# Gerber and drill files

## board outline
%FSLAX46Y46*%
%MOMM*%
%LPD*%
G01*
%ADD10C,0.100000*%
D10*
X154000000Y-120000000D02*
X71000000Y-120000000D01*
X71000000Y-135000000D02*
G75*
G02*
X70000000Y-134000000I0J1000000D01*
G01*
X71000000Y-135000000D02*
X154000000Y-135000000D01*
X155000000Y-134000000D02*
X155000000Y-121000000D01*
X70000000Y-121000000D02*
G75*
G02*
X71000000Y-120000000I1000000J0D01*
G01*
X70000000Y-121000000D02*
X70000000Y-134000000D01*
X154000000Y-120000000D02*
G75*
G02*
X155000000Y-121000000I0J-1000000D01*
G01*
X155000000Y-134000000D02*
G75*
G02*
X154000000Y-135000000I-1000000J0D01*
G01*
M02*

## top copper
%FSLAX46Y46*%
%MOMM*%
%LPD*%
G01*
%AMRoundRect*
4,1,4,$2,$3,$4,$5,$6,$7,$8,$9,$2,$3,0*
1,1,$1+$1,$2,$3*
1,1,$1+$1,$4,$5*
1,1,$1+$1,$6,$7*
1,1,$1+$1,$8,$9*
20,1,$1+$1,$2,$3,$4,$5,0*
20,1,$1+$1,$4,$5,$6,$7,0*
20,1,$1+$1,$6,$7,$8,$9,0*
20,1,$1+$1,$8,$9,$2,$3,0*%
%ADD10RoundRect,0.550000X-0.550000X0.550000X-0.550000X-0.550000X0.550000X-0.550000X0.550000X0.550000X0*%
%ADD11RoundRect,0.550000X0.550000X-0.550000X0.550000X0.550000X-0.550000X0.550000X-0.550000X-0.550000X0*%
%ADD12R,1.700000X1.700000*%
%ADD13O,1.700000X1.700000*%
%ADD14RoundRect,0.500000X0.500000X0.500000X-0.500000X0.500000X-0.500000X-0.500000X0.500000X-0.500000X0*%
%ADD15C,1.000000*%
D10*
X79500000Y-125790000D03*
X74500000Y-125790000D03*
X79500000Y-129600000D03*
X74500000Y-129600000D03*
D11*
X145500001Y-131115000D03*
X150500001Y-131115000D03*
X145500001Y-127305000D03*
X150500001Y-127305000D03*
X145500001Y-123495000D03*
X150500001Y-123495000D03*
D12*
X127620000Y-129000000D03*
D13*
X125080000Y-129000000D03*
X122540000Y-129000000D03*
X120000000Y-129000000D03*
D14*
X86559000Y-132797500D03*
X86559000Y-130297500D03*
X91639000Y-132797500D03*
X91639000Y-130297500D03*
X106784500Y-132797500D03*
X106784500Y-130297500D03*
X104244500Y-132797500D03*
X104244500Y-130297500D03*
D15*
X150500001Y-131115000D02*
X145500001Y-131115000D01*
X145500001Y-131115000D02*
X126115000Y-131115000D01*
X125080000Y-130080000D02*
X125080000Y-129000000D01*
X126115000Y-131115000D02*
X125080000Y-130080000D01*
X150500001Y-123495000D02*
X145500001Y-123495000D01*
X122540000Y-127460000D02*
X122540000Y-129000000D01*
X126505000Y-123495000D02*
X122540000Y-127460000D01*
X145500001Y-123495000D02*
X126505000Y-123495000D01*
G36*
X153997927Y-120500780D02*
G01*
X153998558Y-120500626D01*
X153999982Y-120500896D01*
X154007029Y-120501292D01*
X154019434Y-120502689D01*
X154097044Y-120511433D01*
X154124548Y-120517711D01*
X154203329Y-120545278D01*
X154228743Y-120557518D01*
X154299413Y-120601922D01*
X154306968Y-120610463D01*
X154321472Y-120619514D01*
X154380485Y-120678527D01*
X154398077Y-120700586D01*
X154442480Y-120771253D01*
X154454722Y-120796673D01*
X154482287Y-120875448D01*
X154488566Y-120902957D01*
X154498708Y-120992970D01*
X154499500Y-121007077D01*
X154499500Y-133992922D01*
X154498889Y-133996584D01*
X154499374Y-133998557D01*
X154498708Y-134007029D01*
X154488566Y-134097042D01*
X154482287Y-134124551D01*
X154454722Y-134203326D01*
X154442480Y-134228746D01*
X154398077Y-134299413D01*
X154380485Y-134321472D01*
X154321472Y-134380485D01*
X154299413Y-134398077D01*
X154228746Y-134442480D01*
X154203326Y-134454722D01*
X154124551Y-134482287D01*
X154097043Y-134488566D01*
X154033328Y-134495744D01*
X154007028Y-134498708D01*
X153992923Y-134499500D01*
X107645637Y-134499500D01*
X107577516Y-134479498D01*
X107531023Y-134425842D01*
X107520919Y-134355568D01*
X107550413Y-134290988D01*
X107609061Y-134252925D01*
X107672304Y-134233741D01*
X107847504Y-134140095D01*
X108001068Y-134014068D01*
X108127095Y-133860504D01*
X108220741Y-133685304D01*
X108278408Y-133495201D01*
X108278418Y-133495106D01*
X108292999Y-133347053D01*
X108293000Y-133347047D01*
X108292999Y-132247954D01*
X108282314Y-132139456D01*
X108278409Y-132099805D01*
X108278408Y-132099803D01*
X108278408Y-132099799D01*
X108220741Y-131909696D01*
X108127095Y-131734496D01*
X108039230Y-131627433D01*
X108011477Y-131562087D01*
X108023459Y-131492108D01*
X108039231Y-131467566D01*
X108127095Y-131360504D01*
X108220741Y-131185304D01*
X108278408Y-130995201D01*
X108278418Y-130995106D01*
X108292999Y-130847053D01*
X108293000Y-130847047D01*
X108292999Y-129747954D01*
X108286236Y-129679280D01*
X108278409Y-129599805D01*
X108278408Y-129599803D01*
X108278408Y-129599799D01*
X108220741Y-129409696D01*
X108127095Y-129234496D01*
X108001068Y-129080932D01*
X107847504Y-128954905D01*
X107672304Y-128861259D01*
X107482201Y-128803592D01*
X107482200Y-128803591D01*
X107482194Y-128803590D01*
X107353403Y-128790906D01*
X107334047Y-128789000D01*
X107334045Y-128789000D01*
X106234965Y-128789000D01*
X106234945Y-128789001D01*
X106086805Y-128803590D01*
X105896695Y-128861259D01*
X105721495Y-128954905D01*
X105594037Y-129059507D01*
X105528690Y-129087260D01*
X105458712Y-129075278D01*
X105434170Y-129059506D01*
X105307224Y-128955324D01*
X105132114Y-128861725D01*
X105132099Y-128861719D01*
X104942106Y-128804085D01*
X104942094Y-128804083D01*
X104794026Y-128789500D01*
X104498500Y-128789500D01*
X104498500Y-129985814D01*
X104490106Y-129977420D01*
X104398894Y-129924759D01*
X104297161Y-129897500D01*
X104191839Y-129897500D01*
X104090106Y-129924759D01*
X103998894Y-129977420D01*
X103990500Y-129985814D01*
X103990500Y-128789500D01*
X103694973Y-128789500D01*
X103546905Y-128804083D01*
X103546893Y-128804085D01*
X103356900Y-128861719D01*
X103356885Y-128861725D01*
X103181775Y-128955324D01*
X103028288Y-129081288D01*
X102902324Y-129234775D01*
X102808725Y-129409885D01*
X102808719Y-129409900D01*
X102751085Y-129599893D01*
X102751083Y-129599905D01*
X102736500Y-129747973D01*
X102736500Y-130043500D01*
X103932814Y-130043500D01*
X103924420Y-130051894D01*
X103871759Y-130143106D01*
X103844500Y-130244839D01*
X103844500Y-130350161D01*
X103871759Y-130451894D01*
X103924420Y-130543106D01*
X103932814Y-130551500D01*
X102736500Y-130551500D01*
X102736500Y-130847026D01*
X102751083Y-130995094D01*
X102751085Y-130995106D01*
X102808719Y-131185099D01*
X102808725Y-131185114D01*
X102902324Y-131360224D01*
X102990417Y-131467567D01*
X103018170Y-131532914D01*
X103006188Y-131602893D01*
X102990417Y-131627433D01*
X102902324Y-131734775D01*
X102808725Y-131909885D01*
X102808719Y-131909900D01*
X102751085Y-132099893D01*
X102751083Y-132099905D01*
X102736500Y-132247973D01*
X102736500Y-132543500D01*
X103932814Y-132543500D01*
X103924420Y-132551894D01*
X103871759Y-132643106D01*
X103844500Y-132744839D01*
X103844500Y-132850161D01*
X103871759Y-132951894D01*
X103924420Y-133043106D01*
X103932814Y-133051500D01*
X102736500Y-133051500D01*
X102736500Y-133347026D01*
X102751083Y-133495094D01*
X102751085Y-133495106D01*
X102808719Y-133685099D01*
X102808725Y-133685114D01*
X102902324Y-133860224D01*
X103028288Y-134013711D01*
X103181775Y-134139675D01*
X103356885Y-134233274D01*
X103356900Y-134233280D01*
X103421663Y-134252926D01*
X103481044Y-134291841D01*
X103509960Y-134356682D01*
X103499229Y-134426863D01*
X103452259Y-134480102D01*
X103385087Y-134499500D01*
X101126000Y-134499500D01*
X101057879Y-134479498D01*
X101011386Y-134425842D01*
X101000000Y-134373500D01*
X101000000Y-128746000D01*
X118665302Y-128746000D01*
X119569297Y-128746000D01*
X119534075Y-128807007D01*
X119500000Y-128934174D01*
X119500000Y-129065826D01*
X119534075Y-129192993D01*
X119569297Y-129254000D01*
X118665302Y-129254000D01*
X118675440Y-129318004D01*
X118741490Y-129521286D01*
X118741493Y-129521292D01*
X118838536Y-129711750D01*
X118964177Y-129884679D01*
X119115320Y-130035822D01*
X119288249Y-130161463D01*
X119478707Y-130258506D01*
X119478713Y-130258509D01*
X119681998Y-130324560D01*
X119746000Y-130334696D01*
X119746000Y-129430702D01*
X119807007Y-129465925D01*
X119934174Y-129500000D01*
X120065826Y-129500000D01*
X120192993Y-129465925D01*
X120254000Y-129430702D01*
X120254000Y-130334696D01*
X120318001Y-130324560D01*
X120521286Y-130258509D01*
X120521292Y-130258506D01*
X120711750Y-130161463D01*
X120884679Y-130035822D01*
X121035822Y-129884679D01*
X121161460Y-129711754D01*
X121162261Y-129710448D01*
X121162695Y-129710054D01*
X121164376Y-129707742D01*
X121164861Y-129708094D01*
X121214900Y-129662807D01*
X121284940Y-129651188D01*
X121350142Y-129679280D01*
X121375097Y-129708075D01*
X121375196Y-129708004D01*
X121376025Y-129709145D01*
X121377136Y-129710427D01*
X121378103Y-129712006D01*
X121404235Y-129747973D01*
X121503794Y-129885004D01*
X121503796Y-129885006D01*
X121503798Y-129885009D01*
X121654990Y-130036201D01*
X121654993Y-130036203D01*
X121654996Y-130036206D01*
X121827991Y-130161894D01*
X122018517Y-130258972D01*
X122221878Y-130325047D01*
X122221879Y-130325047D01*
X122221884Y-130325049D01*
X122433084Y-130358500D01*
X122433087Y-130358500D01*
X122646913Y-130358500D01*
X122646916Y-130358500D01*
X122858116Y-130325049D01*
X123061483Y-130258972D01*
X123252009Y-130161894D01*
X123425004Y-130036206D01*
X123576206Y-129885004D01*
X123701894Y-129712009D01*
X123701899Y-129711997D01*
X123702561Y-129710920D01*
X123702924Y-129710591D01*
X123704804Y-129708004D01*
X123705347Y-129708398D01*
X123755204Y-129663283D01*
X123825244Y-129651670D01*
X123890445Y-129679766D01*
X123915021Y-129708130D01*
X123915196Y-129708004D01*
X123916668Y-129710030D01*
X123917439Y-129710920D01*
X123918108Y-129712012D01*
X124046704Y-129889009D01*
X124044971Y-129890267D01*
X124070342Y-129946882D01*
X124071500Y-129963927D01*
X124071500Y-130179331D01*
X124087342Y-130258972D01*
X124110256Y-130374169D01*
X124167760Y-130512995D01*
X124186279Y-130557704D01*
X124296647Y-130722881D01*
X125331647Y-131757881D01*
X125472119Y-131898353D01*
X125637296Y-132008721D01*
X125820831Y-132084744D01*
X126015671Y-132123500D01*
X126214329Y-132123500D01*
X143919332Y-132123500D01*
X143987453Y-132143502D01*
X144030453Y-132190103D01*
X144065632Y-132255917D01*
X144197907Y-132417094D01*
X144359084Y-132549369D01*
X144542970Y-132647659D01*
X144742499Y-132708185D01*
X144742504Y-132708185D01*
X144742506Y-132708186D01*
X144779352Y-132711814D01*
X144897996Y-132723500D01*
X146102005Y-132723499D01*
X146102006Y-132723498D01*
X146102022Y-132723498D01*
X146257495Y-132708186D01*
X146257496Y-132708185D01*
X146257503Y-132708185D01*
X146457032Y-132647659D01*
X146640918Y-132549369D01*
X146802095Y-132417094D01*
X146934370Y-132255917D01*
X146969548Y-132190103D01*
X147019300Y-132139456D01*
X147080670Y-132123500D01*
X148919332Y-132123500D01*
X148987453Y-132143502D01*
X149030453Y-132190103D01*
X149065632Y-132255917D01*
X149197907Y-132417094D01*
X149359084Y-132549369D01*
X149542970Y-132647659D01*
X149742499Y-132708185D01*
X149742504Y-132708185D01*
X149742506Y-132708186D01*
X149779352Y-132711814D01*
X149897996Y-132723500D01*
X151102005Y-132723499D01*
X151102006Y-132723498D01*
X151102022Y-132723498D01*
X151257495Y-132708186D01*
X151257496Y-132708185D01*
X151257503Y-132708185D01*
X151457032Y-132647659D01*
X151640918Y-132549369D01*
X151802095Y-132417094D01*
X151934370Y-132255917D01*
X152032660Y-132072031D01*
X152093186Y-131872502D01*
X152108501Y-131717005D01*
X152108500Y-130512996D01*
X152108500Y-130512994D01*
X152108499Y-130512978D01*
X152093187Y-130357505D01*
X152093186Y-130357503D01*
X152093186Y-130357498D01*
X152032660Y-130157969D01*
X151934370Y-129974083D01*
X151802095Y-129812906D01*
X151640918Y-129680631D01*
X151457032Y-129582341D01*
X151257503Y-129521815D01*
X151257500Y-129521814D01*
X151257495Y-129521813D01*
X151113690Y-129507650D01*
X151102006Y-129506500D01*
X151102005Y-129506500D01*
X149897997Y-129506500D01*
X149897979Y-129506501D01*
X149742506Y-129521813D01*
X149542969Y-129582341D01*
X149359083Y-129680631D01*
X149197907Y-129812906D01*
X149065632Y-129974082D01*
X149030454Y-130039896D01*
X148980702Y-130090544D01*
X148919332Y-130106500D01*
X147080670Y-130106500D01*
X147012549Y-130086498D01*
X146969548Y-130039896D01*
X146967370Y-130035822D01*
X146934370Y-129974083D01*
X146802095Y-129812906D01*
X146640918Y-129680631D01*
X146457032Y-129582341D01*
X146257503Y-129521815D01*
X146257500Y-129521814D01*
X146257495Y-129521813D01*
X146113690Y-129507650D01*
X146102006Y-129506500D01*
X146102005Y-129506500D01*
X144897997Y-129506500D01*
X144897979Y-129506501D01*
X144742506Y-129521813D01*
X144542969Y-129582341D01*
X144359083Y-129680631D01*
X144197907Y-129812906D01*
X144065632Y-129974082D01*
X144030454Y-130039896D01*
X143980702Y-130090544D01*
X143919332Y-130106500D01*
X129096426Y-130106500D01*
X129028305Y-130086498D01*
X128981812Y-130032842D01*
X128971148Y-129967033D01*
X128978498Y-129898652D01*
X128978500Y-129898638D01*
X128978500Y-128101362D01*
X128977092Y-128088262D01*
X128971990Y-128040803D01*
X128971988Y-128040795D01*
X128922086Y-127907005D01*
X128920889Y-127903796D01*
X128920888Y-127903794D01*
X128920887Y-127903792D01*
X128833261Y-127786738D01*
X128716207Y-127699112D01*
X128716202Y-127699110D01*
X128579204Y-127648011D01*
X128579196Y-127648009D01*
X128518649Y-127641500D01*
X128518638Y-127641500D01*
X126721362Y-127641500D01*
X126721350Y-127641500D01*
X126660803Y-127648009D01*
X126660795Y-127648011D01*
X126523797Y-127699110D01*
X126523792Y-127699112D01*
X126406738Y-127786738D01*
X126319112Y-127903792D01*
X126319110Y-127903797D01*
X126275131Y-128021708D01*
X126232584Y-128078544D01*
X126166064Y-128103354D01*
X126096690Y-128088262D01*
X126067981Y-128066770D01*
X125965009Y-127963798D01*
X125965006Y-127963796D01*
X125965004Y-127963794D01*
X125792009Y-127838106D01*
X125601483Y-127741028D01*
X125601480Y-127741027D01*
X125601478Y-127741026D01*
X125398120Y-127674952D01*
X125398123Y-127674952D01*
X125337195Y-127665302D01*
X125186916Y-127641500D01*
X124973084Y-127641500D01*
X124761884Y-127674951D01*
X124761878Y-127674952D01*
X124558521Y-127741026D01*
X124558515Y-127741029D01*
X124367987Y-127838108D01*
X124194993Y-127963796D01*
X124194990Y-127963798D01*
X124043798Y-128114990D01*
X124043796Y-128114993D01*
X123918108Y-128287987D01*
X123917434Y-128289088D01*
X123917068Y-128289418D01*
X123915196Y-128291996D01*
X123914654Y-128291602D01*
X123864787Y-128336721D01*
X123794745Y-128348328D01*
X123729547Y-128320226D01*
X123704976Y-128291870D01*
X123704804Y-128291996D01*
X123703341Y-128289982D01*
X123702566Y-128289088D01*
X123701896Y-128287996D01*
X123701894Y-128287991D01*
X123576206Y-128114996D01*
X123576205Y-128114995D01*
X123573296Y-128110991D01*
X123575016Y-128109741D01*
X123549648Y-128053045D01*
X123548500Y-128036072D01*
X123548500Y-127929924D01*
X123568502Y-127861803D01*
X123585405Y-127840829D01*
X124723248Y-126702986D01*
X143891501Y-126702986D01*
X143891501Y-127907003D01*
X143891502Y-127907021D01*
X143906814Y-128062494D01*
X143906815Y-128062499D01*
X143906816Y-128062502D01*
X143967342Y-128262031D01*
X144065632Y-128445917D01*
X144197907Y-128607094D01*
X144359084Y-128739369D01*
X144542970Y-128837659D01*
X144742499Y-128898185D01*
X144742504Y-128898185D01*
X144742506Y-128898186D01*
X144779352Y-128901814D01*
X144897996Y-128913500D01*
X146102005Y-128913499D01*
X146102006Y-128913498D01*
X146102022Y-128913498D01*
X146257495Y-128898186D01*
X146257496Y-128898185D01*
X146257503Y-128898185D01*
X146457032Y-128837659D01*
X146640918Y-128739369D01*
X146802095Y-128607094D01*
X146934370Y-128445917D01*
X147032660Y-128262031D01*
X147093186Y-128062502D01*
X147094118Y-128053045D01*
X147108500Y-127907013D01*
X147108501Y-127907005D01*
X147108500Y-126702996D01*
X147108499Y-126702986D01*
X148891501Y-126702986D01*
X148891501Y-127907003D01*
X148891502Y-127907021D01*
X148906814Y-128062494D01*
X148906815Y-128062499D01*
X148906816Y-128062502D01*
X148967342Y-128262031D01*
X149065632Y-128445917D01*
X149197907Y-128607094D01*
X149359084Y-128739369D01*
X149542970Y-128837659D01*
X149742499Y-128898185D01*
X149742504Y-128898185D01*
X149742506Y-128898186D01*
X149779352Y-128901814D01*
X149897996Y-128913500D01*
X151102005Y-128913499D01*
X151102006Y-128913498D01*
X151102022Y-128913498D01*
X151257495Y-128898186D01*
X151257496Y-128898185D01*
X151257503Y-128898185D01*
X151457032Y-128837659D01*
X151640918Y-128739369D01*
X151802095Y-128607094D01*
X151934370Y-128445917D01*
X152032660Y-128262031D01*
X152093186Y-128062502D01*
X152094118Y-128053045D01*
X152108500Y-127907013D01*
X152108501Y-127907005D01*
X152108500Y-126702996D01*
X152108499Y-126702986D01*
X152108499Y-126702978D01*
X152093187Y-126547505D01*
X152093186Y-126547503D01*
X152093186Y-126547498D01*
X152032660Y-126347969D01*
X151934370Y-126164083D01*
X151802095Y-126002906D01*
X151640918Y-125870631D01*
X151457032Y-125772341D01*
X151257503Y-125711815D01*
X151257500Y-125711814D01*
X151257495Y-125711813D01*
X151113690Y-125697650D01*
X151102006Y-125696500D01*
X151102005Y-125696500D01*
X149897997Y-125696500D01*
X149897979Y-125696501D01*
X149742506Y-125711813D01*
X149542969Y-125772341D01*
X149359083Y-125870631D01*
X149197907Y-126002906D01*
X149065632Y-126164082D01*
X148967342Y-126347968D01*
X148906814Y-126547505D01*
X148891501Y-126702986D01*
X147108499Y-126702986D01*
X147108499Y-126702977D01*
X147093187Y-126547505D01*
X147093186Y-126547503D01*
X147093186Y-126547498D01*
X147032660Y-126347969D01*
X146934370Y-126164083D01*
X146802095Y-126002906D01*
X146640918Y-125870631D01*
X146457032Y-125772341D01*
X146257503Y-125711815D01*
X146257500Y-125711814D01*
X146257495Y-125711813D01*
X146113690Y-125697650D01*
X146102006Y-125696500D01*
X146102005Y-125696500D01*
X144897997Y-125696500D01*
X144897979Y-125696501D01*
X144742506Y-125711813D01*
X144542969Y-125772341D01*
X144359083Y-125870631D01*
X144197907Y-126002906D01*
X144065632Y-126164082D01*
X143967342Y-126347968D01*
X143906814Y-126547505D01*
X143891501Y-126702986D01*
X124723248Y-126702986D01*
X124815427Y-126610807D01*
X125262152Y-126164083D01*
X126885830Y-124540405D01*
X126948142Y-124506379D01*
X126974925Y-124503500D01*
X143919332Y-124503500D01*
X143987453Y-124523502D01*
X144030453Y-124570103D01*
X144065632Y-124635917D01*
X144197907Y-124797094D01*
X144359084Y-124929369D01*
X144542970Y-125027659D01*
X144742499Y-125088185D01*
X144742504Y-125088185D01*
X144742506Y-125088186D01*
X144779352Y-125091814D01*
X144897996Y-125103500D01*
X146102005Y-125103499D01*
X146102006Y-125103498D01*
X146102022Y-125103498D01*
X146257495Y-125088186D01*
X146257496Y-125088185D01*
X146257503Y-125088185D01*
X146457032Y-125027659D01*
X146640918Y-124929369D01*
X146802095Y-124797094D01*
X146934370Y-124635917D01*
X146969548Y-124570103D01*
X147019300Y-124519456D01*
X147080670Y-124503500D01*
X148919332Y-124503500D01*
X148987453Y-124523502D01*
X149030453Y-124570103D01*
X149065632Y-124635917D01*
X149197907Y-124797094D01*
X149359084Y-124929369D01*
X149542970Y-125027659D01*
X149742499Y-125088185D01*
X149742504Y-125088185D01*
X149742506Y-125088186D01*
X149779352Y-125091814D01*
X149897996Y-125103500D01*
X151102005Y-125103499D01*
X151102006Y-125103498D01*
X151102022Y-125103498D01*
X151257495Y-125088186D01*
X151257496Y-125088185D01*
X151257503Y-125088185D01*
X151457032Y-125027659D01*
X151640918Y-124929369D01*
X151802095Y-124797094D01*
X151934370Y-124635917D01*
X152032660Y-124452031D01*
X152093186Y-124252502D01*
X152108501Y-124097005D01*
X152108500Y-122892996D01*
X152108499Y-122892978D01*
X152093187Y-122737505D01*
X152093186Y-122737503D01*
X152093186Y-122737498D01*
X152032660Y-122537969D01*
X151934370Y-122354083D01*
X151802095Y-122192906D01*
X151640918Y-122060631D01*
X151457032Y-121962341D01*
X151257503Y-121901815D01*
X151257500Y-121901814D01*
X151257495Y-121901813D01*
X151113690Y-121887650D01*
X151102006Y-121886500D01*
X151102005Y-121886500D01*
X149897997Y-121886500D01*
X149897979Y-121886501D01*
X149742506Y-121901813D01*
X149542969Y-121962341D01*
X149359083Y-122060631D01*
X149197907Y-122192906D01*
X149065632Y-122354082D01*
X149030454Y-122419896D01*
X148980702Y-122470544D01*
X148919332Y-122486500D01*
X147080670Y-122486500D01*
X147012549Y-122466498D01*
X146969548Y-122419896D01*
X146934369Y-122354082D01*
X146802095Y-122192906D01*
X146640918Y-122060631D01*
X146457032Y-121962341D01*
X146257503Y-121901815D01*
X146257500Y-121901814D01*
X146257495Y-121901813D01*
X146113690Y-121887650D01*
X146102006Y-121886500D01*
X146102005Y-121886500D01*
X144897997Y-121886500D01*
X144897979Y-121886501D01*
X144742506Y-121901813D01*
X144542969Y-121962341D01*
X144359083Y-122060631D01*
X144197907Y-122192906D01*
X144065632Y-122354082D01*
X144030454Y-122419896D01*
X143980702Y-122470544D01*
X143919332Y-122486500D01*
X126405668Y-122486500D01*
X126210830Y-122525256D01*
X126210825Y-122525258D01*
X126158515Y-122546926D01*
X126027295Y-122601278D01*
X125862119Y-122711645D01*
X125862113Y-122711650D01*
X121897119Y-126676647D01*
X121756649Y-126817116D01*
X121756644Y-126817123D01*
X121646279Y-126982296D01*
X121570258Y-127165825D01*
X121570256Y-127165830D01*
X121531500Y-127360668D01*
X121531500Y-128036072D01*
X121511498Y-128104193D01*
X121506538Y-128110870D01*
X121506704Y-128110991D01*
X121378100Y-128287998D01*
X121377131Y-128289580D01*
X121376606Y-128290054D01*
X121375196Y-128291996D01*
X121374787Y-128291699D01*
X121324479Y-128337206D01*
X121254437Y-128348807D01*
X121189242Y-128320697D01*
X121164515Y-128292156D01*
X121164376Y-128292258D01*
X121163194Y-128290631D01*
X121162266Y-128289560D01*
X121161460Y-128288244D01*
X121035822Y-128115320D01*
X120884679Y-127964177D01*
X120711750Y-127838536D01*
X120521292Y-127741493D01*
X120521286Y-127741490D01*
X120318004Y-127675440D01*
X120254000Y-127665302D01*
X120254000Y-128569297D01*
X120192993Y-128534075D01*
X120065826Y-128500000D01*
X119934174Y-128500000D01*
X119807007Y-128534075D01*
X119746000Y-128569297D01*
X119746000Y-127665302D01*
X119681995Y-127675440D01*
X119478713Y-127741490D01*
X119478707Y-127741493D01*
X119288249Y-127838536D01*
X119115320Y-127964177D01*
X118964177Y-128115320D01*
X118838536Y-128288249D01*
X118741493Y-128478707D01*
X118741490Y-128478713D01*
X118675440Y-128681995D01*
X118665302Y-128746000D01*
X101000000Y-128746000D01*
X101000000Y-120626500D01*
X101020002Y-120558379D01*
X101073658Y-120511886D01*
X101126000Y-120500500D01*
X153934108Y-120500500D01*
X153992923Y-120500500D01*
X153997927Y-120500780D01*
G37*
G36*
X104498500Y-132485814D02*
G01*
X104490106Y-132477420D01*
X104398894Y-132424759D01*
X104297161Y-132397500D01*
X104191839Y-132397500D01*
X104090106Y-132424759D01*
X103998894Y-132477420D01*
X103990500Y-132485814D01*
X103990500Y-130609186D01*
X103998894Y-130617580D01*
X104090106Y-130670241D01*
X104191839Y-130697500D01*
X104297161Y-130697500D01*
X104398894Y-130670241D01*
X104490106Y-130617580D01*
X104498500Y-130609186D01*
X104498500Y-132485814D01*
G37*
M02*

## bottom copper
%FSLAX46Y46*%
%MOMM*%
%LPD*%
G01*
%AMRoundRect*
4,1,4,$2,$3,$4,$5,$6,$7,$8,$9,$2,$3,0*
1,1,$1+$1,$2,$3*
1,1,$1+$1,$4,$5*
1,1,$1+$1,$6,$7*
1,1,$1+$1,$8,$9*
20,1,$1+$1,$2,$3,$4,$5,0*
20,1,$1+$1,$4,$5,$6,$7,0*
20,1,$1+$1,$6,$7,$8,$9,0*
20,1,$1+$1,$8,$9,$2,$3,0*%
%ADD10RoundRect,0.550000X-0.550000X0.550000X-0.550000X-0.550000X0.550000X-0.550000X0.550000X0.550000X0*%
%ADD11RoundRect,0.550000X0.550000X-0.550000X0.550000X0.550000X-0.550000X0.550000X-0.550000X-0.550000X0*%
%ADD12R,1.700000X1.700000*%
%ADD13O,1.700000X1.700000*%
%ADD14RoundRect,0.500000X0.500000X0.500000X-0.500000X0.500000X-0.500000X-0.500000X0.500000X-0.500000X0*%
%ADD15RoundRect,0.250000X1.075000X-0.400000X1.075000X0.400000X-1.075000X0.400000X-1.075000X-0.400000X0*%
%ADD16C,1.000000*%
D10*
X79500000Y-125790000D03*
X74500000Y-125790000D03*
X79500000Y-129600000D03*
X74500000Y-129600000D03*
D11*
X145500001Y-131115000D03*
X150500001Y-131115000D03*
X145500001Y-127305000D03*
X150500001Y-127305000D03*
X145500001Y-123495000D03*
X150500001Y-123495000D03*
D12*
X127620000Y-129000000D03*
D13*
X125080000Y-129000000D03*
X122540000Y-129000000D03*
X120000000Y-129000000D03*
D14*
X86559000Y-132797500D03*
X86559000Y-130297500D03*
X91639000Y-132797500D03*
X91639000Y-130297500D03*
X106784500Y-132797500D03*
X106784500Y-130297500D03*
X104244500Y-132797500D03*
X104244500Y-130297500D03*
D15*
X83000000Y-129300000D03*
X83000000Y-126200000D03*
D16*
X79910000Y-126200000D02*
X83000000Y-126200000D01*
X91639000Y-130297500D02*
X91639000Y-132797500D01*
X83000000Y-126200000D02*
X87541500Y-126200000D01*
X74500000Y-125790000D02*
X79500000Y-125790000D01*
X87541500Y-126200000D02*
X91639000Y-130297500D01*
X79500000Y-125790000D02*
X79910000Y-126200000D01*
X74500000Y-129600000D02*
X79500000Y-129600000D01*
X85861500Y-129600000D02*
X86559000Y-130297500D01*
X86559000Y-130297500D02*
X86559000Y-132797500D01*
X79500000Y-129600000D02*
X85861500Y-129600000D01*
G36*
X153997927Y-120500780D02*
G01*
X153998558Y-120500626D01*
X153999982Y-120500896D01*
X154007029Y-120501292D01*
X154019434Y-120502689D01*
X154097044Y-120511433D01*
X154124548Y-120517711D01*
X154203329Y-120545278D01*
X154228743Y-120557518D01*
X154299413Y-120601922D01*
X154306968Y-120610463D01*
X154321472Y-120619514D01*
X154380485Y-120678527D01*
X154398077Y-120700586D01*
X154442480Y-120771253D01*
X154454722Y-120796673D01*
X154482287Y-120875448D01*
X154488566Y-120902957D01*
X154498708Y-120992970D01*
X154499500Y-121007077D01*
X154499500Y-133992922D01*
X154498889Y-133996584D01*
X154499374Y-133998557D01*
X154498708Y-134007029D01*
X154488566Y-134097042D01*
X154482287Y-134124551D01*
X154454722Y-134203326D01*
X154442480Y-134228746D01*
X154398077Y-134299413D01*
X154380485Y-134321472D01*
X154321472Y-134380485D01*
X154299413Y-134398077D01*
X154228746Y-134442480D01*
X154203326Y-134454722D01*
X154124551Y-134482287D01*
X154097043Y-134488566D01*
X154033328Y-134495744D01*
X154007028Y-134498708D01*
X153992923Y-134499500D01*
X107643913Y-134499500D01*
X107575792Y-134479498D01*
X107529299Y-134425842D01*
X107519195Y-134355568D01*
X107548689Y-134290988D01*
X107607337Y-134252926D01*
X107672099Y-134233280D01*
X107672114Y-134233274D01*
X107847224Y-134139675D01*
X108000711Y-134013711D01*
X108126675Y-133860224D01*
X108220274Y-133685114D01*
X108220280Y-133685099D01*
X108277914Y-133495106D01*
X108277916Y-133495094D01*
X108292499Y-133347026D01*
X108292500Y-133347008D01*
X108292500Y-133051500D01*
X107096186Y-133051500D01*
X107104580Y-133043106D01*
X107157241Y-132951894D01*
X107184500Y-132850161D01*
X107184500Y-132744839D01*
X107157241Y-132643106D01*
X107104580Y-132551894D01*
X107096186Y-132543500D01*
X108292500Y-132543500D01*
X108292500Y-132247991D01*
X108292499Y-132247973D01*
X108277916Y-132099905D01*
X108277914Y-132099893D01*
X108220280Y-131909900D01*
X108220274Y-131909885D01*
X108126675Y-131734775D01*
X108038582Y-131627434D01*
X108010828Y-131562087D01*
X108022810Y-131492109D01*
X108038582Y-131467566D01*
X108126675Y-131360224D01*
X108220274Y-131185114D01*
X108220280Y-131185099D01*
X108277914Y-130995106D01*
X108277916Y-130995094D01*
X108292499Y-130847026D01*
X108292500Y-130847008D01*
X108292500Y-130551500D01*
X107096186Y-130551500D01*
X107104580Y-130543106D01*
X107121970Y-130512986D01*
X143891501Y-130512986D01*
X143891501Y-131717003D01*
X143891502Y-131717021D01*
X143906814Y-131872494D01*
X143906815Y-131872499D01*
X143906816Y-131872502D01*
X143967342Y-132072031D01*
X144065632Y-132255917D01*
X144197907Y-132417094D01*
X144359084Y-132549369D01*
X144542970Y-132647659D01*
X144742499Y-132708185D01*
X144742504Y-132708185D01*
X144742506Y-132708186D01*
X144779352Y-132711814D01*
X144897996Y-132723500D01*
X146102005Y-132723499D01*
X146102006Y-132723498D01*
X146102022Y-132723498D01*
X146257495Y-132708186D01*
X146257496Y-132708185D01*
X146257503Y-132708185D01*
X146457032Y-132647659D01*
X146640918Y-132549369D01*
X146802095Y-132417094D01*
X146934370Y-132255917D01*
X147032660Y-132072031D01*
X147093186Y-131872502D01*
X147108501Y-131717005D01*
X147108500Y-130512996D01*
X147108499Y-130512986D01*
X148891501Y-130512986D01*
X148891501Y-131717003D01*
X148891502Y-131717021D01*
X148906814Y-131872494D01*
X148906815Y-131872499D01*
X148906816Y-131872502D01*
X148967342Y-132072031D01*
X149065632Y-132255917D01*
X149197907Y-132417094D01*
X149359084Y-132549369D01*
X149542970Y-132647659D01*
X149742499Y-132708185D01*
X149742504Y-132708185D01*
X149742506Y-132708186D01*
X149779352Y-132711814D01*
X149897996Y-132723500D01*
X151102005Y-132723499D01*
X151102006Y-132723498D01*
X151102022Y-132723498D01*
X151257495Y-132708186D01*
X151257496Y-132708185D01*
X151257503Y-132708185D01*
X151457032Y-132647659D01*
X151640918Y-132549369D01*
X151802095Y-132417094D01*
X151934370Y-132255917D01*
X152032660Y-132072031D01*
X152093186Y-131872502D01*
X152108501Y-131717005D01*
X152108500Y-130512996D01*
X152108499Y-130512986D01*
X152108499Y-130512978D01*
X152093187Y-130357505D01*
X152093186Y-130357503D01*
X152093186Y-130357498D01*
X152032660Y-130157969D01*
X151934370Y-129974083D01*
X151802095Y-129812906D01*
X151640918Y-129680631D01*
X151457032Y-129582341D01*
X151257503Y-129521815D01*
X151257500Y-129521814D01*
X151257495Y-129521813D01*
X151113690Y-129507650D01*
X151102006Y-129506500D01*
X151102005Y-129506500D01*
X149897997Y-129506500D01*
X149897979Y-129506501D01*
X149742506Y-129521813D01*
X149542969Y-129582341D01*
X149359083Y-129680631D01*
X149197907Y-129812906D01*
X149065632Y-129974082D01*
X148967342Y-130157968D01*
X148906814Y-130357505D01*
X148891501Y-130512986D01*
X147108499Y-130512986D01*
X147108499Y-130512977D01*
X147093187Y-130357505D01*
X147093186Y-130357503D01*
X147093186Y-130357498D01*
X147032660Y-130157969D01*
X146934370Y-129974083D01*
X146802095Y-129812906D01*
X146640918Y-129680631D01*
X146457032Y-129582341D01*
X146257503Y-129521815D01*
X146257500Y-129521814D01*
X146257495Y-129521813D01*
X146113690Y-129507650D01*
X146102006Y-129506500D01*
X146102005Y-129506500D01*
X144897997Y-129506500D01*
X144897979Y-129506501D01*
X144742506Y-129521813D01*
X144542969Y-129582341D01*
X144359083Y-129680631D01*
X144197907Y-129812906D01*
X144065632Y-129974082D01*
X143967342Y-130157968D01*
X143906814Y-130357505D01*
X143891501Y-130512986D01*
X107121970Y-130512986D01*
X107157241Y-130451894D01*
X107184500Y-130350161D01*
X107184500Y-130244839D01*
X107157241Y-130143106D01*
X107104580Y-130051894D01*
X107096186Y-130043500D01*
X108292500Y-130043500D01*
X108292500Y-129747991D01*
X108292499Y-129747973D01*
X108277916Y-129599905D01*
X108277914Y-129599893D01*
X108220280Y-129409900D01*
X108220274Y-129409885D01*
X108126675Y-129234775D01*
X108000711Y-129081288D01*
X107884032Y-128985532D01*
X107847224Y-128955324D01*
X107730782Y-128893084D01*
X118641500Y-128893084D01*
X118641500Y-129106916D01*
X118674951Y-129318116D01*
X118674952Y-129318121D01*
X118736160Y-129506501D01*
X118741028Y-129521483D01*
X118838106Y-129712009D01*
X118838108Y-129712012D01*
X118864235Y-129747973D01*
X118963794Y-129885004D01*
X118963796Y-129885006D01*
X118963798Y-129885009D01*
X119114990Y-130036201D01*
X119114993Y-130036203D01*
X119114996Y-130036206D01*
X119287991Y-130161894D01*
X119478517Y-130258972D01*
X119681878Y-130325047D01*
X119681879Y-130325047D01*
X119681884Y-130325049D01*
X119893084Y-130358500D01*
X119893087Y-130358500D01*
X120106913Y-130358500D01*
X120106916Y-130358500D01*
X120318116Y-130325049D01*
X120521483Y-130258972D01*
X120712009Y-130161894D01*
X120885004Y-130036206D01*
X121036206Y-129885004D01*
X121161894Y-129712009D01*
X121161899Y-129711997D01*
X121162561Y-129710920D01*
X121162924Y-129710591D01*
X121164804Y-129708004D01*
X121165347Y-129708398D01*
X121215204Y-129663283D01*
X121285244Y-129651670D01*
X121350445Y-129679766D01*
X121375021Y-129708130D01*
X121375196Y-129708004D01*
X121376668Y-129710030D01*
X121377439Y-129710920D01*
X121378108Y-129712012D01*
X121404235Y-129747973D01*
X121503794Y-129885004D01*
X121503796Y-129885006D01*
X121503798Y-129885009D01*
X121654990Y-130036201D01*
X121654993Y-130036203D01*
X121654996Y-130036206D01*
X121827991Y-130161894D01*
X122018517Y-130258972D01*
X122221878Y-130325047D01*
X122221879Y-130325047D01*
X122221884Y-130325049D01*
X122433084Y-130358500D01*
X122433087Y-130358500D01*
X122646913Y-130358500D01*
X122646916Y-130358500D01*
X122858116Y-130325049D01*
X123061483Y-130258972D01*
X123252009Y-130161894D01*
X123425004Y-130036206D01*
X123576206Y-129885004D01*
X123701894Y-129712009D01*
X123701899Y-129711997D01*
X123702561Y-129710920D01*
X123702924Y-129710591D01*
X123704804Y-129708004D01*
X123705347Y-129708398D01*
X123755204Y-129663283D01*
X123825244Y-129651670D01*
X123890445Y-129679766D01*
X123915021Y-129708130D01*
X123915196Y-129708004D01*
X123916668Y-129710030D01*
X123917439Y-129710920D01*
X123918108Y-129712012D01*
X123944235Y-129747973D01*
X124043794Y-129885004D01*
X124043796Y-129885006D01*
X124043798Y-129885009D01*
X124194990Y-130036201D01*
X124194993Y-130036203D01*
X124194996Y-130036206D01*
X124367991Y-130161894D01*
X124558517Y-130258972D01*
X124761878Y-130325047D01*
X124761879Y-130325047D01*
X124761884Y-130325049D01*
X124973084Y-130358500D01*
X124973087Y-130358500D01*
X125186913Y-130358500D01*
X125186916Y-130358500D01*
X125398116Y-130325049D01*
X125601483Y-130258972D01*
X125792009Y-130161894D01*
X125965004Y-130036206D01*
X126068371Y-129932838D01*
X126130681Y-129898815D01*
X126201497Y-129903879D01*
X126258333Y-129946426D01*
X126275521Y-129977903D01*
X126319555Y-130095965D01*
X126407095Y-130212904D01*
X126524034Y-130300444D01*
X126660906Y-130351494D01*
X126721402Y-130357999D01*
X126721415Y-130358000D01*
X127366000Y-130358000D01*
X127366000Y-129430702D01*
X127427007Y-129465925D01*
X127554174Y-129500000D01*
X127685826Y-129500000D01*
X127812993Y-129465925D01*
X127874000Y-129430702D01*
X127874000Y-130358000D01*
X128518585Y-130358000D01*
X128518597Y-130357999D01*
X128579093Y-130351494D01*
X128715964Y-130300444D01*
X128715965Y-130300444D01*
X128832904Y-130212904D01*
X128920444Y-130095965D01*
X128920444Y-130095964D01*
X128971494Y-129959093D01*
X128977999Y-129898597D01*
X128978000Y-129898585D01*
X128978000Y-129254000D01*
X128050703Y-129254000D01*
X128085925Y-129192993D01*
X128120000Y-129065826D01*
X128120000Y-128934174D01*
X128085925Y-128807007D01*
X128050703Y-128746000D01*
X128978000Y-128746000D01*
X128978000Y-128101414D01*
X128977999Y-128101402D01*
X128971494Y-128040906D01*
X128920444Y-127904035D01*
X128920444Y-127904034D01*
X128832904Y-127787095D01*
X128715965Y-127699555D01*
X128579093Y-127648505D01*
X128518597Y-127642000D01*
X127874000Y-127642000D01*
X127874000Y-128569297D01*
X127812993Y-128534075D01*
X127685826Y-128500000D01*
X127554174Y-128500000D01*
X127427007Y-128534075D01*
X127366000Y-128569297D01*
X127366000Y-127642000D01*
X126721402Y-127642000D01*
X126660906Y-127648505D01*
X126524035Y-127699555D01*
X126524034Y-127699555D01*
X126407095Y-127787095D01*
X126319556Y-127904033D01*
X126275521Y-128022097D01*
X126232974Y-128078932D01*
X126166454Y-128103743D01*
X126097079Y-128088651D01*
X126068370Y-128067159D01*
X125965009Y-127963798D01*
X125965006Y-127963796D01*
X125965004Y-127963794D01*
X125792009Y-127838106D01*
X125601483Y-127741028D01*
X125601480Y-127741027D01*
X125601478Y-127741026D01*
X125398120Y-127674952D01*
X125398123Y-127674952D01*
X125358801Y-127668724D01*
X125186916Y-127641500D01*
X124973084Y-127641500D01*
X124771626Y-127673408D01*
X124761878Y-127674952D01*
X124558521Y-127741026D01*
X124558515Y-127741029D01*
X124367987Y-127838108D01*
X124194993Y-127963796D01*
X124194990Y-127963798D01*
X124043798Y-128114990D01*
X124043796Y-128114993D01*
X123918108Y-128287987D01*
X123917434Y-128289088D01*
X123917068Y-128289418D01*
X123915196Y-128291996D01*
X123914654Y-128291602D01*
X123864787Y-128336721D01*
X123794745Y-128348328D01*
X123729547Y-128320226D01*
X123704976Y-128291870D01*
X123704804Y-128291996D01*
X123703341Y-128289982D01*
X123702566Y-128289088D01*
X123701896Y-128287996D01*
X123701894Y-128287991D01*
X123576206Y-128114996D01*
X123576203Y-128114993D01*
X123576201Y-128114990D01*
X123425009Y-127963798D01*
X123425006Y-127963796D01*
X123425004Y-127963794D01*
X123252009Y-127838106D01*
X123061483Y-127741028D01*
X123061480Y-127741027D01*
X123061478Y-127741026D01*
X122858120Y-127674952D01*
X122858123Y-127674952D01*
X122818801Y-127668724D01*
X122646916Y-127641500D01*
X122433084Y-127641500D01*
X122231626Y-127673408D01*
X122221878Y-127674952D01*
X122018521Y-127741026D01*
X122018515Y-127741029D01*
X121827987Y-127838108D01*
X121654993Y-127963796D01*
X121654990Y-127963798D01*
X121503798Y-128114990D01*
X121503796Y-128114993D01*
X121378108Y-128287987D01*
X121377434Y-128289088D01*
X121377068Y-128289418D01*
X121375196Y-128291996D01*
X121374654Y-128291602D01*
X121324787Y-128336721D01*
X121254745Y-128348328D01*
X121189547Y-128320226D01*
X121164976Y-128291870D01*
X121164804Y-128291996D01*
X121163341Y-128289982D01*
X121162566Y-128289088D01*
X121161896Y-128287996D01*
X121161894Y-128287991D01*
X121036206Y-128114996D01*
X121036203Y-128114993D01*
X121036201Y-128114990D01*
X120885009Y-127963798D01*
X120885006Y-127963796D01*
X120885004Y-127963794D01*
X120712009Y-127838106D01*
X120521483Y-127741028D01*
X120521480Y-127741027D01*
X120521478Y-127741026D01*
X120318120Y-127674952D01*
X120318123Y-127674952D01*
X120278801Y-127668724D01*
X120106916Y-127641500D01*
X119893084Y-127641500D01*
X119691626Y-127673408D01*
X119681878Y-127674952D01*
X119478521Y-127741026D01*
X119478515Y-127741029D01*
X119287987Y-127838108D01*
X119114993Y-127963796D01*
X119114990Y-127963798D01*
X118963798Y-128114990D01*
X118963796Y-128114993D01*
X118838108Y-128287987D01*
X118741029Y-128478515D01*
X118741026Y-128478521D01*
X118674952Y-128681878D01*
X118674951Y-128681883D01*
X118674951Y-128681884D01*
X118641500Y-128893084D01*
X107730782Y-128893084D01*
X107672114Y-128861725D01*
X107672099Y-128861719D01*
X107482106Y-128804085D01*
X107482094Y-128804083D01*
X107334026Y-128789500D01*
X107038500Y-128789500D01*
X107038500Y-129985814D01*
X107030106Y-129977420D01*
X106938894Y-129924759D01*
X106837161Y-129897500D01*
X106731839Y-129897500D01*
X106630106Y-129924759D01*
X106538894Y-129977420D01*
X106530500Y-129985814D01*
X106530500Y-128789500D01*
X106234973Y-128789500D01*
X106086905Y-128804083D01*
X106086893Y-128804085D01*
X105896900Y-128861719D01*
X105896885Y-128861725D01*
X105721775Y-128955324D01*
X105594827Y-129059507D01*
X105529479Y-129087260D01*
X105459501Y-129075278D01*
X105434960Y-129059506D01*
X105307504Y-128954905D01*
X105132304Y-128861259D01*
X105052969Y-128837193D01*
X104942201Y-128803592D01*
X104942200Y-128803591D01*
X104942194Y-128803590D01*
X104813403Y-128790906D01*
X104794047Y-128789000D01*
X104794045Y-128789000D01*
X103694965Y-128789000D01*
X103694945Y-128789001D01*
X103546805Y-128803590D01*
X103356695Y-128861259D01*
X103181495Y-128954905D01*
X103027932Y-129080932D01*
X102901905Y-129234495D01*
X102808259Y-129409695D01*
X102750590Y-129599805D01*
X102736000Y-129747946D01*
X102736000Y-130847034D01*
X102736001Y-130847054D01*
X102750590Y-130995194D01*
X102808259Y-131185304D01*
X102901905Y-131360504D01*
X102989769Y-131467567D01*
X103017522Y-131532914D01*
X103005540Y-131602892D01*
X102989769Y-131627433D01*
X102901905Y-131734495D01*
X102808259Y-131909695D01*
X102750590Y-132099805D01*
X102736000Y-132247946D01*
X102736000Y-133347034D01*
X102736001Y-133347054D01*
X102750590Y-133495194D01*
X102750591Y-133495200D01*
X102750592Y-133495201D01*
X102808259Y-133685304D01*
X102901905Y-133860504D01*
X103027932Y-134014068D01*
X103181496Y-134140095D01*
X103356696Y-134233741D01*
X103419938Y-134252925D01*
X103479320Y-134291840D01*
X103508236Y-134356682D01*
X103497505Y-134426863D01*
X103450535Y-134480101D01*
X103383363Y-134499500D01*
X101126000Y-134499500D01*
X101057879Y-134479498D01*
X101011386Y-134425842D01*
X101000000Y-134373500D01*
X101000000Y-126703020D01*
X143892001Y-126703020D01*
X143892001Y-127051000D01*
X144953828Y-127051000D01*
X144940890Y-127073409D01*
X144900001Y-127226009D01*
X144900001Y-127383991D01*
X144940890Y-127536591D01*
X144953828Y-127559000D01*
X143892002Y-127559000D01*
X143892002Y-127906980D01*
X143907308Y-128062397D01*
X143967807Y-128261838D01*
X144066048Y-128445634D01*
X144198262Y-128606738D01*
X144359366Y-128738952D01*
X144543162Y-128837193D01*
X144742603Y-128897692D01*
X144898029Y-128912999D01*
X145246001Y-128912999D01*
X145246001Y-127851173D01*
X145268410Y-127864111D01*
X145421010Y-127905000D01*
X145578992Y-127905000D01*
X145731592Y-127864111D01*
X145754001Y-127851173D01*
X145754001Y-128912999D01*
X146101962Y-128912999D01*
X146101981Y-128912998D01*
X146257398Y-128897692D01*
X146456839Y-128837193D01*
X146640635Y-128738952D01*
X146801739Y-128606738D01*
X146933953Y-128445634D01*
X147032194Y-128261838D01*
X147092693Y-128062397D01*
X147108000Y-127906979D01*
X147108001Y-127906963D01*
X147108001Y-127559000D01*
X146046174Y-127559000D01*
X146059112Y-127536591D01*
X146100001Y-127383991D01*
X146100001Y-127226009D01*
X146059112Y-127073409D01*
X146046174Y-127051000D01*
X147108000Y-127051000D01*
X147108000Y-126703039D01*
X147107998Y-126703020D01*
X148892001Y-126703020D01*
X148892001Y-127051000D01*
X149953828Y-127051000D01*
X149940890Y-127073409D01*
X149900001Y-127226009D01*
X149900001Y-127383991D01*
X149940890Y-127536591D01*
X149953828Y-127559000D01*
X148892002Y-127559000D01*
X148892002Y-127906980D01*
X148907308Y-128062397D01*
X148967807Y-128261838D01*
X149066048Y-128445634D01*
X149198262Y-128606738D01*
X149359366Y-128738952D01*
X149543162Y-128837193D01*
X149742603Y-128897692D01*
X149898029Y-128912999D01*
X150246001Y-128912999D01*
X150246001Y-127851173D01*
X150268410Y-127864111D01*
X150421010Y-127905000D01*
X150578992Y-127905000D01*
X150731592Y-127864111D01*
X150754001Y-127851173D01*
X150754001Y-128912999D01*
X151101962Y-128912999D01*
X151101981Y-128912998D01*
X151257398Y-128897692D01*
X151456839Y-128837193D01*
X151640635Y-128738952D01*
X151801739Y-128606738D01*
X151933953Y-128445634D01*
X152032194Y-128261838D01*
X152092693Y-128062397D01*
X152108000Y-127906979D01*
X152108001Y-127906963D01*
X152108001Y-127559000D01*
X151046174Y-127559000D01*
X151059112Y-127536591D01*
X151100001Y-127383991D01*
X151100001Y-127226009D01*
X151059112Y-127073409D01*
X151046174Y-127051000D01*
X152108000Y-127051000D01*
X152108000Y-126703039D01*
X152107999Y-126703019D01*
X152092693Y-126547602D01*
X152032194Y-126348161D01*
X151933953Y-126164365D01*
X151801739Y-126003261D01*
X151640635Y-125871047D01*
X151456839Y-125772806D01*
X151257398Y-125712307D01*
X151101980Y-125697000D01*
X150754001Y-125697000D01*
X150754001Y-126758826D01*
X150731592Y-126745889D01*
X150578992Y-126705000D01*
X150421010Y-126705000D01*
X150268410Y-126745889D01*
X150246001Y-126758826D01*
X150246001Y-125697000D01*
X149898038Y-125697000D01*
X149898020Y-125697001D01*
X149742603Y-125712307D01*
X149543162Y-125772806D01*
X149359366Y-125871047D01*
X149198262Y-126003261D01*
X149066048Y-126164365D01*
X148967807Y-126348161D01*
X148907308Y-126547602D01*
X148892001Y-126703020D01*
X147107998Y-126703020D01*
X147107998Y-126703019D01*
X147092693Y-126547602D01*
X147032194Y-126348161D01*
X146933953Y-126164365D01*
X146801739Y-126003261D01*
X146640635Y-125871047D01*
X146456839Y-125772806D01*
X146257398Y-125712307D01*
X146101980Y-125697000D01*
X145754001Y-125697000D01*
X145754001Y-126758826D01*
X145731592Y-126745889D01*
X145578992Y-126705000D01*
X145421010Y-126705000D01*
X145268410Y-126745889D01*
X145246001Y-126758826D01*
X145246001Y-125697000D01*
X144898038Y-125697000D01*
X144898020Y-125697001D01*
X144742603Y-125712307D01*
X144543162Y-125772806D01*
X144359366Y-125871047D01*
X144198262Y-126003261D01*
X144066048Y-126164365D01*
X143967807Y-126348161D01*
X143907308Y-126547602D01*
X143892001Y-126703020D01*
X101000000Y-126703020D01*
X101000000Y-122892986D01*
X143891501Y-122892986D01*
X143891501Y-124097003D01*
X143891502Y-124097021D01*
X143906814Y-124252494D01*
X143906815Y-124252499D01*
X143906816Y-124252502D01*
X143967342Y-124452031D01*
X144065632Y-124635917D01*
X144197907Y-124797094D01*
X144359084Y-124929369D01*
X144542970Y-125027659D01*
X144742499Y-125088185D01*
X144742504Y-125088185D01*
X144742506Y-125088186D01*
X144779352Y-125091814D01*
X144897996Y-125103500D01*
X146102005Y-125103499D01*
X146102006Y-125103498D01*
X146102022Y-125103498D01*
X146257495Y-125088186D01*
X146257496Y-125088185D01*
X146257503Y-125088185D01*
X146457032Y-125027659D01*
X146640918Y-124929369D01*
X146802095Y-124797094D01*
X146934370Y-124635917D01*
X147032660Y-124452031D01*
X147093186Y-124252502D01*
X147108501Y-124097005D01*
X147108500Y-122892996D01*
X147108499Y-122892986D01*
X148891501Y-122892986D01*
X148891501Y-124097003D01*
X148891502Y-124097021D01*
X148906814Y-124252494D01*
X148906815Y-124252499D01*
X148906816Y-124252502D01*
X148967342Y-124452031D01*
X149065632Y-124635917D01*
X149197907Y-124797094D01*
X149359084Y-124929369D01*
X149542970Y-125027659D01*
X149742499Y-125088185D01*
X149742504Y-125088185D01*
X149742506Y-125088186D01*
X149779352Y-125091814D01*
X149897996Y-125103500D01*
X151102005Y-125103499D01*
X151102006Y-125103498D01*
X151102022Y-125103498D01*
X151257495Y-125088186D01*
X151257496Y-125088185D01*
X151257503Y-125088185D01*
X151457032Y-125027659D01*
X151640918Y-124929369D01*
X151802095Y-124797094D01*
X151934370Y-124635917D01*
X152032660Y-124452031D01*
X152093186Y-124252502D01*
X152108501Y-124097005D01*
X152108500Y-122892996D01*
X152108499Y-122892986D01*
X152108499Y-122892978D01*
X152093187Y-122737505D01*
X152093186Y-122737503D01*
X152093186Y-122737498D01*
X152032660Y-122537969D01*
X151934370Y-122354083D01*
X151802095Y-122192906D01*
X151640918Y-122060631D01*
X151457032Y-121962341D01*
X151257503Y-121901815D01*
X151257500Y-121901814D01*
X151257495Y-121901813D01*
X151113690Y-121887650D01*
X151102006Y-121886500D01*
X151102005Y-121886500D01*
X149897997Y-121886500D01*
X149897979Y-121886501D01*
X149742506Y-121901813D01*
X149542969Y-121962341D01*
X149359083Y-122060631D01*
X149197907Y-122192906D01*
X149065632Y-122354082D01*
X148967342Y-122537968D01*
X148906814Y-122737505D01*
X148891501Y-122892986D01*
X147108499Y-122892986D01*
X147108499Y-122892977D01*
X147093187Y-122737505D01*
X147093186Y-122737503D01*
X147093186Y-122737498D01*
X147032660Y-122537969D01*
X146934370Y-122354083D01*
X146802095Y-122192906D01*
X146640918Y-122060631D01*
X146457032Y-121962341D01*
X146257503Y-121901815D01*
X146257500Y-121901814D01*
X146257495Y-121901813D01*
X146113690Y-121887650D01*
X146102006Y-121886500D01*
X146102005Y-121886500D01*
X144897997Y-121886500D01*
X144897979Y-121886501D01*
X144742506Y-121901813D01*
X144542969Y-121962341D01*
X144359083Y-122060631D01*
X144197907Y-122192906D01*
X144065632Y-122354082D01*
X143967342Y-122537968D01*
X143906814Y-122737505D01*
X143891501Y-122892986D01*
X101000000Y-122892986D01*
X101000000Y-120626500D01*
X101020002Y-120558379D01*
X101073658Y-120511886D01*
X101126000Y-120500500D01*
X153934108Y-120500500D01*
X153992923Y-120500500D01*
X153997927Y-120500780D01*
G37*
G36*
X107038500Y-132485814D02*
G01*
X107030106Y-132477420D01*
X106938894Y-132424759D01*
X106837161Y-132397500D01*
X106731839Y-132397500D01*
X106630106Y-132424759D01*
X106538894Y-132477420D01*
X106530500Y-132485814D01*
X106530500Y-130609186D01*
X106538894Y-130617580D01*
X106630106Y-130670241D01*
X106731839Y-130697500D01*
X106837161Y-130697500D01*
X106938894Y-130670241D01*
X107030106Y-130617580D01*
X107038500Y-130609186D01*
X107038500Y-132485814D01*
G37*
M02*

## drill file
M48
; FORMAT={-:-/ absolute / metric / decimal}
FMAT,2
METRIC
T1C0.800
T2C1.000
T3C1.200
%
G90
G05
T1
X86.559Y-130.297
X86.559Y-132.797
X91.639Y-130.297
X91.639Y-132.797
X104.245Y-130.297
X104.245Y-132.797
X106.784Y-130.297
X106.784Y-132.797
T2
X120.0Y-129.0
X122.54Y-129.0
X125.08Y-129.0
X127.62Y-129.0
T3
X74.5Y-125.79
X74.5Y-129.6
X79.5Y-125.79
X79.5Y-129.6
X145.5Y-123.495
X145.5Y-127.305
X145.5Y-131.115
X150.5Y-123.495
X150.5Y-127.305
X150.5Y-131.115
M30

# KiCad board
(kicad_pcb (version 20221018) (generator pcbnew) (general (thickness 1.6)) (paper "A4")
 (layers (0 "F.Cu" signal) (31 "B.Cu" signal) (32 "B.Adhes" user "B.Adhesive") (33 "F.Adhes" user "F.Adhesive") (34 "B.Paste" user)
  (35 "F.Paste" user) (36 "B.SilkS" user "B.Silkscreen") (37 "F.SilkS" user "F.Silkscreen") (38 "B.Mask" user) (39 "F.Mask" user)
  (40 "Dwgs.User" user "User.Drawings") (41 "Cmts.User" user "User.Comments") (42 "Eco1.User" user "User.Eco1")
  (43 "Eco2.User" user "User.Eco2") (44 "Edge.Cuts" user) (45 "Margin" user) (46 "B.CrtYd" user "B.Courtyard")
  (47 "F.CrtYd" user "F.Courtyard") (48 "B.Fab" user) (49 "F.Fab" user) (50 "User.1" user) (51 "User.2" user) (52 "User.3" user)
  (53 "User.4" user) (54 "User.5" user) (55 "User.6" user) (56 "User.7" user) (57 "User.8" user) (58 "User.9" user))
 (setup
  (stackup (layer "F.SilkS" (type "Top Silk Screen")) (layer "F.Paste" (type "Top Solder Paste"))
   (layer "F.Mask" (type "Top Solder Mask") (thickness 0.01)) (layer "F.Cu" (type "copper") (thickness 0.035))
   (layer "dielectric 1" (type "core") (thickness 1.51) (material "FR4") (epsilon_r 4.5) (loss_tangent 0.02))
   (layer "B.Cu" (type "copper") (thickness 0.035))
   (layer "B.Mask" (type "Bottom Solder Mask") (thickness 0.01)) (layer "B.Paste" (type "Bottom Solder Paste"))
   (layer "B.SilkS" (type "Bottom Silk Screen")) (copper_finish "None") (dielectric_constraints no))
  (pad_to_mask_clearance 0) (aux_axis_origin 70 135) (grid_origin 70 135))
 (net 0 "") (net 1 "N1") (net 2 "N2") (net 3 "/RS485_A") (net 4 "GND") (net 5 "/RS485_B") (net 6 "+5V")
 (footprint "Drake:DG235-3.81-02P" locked (layer "F.Cu") (at 79.5 125.79 -90)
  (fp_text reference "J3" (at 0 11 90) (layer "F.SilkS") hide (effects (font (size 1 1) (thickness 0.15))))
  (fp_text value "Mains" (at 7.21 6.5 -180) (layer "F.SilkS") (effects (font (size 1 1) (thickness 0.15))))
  (pad "1" thru_hole roundrect locked (at 0 0 270) (size 2.2 2.2) (drill 1.2) (layers "*.Cu" "*.Mask") (roundrect_rratio 0.25) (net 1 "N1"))
  (pad "1" thru_hole roundrect locked (at 0 5 270) (size 2.2 2.2) (drill 1.2) (layers "*.Cu" "*.Mask") (roundrect_rratio 0.25) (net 1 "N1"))
  (pad "2" thru_hole roundrect locked (at 3.81 0 270) (size 2.2 2.2) (drill 1.2) (layers "*.Cu" "*.Mask") (roundrect_rratio 0.25)
   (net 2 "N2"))
  (pad "2" thru_hole roundrect locked (at 3.81 5 270) (size 2.2 2.2) (drill 1.2) (layers "*.Cu" "*.Mask") (roundrect_rratio 0.25)
   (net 2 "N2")))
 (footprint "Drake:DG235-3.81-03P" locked (layer "F.Cu") (at 145.500001 131.115 90)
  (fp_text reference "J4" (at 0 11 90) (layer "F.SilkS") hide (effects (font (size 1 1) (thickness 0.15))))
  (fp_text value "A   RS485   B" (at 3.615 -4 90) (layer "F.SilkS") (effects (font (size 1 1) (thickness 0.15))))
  (pad "1" thru_hole roundrect locked (at 0 0 90) (size 2.2 2.2) (drill 1.2) (layers "*.Cu" "*.Mask") (roundrect_rratio 0.25)
   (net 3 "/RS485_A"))
  (pad "1" thru_hole roundrect locked (at 0 5 90) (size 2.2 2.2) (drill 1.2) (layers "*.Cu" "*.Mask") (roundrect_rratio 0.25)
   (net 3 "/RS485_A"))
  (pad "2" thru_hole roundrect locked (at 3.81 0 90) (size 2.2 2.2) (drill 1.2) (layers "*.Cu" "*.Mask") (roundrect_rratio 0.25)
   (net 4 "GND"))
  (pad "2" thru_hole roundrect locked (at 3.81 5 90) (size 2.2 2.2) (drill 1.2) (layers "*.Cu" "*.Mask") (roundrect_rratio 0.25)
   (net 4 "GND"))
  (pad "3" thru_hole roundrect locked (at 7.62 0 90) (size 2.2 2.2) (drill 1.2) (layers "*.Cu" "*.Mask") (roundrect_rratio 0.25)
   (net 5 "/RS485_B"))
  (pad "3" thru_hole roundrect locked (at 7.62 5 90) (size 2.2 2.2) (drill 1.2) (layers "*.Cu" "*.Mask") (roundrect_rratio 0.25)
   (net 5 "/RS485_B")))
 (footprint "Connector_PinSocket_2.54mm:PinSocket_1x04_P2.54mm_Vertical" (layer "F.Cu") (at 127.62 129 -90)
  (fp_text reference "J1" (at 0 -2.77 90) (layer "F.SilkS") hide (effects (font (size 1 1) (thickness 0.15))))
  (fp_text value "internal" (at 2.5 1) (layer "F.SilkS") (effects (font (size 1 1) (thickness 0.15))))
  (pad "1" thru_hole rect (at 0 0 270) (size 1.7 1.7) (drill 1) (layers "*.Cu" "*.Mask") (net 4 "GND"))
  (pad "2" thru_hole oval (at 0 2.54 270) (size 1.7 1.7) (drill 1) (layers "*.Cu" "*.Mask") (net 3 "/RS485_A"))
  (pad "3" thru_hole oval (at 0 5.08 270) (size 1.7 1.7) (drill 1) (layers "*.Cu" "*.Mask") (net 5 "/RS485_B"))
  (pad "4" thru_hole oval (at 0 7.62 270) (size 1.7 1.7) (drill 1) (layers "*.Cu" "*.Mask") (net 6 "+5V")))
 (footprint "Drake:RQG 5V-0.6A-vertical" (layer "F.Cu") (at 85.325 110.4525 180)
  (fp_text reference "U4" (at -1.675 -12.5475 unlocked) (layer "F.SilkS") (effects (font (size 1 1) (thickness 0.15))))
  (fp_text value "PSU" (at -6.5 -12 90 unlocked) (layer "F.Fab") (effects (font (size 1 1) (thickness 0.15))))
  (pad "1" thru_hole roundrect (at -1.234 -22.345 180) (size 2 2) (drill 0.8) (layers "*.Cu" "*.Mask") (roundrect_rratio 0.25) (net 2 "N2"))
  (pad "1" thru_hole roundrect (at -1.234 -19.845 180) (size 2 2) (drill 0.8) (layers "*.Cu" "*.Mask") (roundrect_rratio 0.25) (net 2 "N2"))
  (pad "2" thru_hole roundrect (at -6.314 -22.345 180) (size 2 2) (drill 0.8) (layers "*.Cu" "*.Mask") (roundrect_rratio 0.25) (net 1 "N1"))
  (pad "2" thru_hole roundrect (at -6.314 -19.845 180) (size 2 2) (drill 0.8) (layers "*.Cu" "*.Mask") (roundrect_rratio 0.25) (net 1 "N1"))
  (pad "3" thru_hole roundrect (at -21.4595 -22.345 180) (size 2 2) (drill 0.8) (layers "*.Cu" "*.Mask") (roundrect_rratio 0.25)
   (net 4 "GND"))
  (pad "3" thru_hole roundrect (at -21.4595 -19.845 180) (size 2 2) (drill 0.8) (layers "*.Cu" "*.Mask") (roundrect_rratio 0.25)
   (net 4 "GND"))
  (pad "4" thru_hole roundrect (at -18.9195 -22.345 180) (size 2 2) (drill 0.8) (layers "*.Cu" "*.Mask") (roundrect_rratio 0.25)
   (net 6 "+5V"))
  (pad "4" thru_hole roundrect (at -18.9195 -19.845 180) (size 2 2) (drill 0.8) (layers "*.Cu" "*.Mask") (roundrect_rratio 0.25)
   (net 6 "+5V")))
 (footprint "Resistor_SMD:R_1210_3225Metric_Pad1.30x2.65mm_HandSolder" (layer "B.Cu") (at 83 127.75 90)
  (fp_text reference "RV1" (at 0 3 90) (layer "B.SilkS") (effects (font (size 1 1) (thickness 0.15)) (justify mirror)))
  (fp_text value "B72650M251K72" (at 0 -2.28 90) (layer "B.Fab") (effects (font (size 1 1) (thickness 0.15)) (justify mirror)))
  (pad "1" smd roundrect (at -1.55 0 90) (size 1.3 2.65) (layers "B.Cu" "B.Paste" "B.Mask") (roundrect_rratio 0.1923076923) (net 2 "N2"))
  (pad "2" smd roundrect (at 1.55 0 90) (size 1.3 2.65) (layers "B.Cu" "B.Paste" "B.Mask") (roundrect_rratio 0.1923076923) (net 1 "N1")))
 (gr_line (start 154 120) (end 71 120) (stroke (width 0.1) (type default)) (layer "Edge.Cuts"))
 (gr_arc (start 71 135) (mid 70.292893 134.707107) (end 70 134) (stroke (width 0.1) (type default)) (layer "Edge.Cuts"))
 (gr_line (start 71 135) (end 154 135) (stroke (width 0.1) (type default)) (layer "Edge.Cuts"))
 (gr_line (start 155 134) (end 155 121) (stroke (width 0.1) (type default)) (layer "Edge.Cuts"))
 (gr_arc (start 70 121) (mid 70.292893 120.292893) (end 71 120) (stroke (width 0.1) (type default)) (layer "Edge.Cuts"))
 (gr_line (start 70 121) (end 70 134) (stroke (width 0.1) (type default)) (layer "Edge.Cuts"))
 (gr_arc (start 154 120) (mid 154.707107 120.292893) (end 155 121) (stroke (width 0.1) (type default)) (layer "Edge.Cuts"))
 (gr_arc (start 155 134) (mid 154.707107 134.707107) (end 154 135) (stroke (width 0.1) (type default)) (layer "Edge.Cuts"))
 (segment (start 79.91 126.2) (end 83 126.2) (width 1) (layer "B.Cu") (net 1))
 (segment (start 91.639 130.2975) (end 91.639 132.7975) (width 1) (layer "B.Cu") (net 1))
 (segment (start 83 126.2) (end 87.5415 126.2) (width 1) (layer "B.Cu") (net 1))
 (segment (start 74.5 125.79) (end 79.5 125.79) (width 1) (layer "B.Cu") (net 1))
 (segment (start 87.5415 126.2) (end 91.639 130.2975) (width 1) (layer "B.Cu") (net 1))
 (segment (start 79.5 125.79) (end 79.91 126.2) (width 1) (layer "B.Cu") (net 1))
 (segment (start 74.5 129.6) (end 79.5 129.6) (width 1) (layer "B.Cu") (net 2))
 (segment (start 85.8615 129.6) (end 86.559 130.2975) (width 1) (layer "B.Cu") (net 2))
 (segment (start 86.559 130.2975) (end 86.559 132.7975) (width 1) (layer "B.Cu") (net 2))
 (segment (start 79.5 129.6) (end 85.8615 129.6) (width 1) (layer "B.Cu") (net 2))
 (segment (start 150.500001 131.115) (end 145.500001 131.115) (width 1) (layer "F.Cu") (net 3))
 (segment (start 145.500001 131.115) (end 126.115 131.115) (width 1) (layer "F.Cu") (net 3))
 (segment (start 125.08 130.08) (end 125.08 129) (width 1) (layer "F.Cu") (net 3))
 (segment (start 126.115 131.115) (end 125.08 130.08) (width 1) (layer "F.Cu") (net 3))
 (segment (start 150.500001 123.495) (end 145.500001 123.495) (width 1) (layer "F.Cu") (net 5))
 (segment (start 122.54 127.46) (end 122.54 129) (width 1) (layer "F.Cu") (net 5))
 (segment (start 126.505 123.495) (end 122.54 127.46) (width 1) (layer "F.Cu") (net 5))
 (segment (start 145.500001 123.495) (end 126.505 123.495) (width 1) (layer "F.Cu") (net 5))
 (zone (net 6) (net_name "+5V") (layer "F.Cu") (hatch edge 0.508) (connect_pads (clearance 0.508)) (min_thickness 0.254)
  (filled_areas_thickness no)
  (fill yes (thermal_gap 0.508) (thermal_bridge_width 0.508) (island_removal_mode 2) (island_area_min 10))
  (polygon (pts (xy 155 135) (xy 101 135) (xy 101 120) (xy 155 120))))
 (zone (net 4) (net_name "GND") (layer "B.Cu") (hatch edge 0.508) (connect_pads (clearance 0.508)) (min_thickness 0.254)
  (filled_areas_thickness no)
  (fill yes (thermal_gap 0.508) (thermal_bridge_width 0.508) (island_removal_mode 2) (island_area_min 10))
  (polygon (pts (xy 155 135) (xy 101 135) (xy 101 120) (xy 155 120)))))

